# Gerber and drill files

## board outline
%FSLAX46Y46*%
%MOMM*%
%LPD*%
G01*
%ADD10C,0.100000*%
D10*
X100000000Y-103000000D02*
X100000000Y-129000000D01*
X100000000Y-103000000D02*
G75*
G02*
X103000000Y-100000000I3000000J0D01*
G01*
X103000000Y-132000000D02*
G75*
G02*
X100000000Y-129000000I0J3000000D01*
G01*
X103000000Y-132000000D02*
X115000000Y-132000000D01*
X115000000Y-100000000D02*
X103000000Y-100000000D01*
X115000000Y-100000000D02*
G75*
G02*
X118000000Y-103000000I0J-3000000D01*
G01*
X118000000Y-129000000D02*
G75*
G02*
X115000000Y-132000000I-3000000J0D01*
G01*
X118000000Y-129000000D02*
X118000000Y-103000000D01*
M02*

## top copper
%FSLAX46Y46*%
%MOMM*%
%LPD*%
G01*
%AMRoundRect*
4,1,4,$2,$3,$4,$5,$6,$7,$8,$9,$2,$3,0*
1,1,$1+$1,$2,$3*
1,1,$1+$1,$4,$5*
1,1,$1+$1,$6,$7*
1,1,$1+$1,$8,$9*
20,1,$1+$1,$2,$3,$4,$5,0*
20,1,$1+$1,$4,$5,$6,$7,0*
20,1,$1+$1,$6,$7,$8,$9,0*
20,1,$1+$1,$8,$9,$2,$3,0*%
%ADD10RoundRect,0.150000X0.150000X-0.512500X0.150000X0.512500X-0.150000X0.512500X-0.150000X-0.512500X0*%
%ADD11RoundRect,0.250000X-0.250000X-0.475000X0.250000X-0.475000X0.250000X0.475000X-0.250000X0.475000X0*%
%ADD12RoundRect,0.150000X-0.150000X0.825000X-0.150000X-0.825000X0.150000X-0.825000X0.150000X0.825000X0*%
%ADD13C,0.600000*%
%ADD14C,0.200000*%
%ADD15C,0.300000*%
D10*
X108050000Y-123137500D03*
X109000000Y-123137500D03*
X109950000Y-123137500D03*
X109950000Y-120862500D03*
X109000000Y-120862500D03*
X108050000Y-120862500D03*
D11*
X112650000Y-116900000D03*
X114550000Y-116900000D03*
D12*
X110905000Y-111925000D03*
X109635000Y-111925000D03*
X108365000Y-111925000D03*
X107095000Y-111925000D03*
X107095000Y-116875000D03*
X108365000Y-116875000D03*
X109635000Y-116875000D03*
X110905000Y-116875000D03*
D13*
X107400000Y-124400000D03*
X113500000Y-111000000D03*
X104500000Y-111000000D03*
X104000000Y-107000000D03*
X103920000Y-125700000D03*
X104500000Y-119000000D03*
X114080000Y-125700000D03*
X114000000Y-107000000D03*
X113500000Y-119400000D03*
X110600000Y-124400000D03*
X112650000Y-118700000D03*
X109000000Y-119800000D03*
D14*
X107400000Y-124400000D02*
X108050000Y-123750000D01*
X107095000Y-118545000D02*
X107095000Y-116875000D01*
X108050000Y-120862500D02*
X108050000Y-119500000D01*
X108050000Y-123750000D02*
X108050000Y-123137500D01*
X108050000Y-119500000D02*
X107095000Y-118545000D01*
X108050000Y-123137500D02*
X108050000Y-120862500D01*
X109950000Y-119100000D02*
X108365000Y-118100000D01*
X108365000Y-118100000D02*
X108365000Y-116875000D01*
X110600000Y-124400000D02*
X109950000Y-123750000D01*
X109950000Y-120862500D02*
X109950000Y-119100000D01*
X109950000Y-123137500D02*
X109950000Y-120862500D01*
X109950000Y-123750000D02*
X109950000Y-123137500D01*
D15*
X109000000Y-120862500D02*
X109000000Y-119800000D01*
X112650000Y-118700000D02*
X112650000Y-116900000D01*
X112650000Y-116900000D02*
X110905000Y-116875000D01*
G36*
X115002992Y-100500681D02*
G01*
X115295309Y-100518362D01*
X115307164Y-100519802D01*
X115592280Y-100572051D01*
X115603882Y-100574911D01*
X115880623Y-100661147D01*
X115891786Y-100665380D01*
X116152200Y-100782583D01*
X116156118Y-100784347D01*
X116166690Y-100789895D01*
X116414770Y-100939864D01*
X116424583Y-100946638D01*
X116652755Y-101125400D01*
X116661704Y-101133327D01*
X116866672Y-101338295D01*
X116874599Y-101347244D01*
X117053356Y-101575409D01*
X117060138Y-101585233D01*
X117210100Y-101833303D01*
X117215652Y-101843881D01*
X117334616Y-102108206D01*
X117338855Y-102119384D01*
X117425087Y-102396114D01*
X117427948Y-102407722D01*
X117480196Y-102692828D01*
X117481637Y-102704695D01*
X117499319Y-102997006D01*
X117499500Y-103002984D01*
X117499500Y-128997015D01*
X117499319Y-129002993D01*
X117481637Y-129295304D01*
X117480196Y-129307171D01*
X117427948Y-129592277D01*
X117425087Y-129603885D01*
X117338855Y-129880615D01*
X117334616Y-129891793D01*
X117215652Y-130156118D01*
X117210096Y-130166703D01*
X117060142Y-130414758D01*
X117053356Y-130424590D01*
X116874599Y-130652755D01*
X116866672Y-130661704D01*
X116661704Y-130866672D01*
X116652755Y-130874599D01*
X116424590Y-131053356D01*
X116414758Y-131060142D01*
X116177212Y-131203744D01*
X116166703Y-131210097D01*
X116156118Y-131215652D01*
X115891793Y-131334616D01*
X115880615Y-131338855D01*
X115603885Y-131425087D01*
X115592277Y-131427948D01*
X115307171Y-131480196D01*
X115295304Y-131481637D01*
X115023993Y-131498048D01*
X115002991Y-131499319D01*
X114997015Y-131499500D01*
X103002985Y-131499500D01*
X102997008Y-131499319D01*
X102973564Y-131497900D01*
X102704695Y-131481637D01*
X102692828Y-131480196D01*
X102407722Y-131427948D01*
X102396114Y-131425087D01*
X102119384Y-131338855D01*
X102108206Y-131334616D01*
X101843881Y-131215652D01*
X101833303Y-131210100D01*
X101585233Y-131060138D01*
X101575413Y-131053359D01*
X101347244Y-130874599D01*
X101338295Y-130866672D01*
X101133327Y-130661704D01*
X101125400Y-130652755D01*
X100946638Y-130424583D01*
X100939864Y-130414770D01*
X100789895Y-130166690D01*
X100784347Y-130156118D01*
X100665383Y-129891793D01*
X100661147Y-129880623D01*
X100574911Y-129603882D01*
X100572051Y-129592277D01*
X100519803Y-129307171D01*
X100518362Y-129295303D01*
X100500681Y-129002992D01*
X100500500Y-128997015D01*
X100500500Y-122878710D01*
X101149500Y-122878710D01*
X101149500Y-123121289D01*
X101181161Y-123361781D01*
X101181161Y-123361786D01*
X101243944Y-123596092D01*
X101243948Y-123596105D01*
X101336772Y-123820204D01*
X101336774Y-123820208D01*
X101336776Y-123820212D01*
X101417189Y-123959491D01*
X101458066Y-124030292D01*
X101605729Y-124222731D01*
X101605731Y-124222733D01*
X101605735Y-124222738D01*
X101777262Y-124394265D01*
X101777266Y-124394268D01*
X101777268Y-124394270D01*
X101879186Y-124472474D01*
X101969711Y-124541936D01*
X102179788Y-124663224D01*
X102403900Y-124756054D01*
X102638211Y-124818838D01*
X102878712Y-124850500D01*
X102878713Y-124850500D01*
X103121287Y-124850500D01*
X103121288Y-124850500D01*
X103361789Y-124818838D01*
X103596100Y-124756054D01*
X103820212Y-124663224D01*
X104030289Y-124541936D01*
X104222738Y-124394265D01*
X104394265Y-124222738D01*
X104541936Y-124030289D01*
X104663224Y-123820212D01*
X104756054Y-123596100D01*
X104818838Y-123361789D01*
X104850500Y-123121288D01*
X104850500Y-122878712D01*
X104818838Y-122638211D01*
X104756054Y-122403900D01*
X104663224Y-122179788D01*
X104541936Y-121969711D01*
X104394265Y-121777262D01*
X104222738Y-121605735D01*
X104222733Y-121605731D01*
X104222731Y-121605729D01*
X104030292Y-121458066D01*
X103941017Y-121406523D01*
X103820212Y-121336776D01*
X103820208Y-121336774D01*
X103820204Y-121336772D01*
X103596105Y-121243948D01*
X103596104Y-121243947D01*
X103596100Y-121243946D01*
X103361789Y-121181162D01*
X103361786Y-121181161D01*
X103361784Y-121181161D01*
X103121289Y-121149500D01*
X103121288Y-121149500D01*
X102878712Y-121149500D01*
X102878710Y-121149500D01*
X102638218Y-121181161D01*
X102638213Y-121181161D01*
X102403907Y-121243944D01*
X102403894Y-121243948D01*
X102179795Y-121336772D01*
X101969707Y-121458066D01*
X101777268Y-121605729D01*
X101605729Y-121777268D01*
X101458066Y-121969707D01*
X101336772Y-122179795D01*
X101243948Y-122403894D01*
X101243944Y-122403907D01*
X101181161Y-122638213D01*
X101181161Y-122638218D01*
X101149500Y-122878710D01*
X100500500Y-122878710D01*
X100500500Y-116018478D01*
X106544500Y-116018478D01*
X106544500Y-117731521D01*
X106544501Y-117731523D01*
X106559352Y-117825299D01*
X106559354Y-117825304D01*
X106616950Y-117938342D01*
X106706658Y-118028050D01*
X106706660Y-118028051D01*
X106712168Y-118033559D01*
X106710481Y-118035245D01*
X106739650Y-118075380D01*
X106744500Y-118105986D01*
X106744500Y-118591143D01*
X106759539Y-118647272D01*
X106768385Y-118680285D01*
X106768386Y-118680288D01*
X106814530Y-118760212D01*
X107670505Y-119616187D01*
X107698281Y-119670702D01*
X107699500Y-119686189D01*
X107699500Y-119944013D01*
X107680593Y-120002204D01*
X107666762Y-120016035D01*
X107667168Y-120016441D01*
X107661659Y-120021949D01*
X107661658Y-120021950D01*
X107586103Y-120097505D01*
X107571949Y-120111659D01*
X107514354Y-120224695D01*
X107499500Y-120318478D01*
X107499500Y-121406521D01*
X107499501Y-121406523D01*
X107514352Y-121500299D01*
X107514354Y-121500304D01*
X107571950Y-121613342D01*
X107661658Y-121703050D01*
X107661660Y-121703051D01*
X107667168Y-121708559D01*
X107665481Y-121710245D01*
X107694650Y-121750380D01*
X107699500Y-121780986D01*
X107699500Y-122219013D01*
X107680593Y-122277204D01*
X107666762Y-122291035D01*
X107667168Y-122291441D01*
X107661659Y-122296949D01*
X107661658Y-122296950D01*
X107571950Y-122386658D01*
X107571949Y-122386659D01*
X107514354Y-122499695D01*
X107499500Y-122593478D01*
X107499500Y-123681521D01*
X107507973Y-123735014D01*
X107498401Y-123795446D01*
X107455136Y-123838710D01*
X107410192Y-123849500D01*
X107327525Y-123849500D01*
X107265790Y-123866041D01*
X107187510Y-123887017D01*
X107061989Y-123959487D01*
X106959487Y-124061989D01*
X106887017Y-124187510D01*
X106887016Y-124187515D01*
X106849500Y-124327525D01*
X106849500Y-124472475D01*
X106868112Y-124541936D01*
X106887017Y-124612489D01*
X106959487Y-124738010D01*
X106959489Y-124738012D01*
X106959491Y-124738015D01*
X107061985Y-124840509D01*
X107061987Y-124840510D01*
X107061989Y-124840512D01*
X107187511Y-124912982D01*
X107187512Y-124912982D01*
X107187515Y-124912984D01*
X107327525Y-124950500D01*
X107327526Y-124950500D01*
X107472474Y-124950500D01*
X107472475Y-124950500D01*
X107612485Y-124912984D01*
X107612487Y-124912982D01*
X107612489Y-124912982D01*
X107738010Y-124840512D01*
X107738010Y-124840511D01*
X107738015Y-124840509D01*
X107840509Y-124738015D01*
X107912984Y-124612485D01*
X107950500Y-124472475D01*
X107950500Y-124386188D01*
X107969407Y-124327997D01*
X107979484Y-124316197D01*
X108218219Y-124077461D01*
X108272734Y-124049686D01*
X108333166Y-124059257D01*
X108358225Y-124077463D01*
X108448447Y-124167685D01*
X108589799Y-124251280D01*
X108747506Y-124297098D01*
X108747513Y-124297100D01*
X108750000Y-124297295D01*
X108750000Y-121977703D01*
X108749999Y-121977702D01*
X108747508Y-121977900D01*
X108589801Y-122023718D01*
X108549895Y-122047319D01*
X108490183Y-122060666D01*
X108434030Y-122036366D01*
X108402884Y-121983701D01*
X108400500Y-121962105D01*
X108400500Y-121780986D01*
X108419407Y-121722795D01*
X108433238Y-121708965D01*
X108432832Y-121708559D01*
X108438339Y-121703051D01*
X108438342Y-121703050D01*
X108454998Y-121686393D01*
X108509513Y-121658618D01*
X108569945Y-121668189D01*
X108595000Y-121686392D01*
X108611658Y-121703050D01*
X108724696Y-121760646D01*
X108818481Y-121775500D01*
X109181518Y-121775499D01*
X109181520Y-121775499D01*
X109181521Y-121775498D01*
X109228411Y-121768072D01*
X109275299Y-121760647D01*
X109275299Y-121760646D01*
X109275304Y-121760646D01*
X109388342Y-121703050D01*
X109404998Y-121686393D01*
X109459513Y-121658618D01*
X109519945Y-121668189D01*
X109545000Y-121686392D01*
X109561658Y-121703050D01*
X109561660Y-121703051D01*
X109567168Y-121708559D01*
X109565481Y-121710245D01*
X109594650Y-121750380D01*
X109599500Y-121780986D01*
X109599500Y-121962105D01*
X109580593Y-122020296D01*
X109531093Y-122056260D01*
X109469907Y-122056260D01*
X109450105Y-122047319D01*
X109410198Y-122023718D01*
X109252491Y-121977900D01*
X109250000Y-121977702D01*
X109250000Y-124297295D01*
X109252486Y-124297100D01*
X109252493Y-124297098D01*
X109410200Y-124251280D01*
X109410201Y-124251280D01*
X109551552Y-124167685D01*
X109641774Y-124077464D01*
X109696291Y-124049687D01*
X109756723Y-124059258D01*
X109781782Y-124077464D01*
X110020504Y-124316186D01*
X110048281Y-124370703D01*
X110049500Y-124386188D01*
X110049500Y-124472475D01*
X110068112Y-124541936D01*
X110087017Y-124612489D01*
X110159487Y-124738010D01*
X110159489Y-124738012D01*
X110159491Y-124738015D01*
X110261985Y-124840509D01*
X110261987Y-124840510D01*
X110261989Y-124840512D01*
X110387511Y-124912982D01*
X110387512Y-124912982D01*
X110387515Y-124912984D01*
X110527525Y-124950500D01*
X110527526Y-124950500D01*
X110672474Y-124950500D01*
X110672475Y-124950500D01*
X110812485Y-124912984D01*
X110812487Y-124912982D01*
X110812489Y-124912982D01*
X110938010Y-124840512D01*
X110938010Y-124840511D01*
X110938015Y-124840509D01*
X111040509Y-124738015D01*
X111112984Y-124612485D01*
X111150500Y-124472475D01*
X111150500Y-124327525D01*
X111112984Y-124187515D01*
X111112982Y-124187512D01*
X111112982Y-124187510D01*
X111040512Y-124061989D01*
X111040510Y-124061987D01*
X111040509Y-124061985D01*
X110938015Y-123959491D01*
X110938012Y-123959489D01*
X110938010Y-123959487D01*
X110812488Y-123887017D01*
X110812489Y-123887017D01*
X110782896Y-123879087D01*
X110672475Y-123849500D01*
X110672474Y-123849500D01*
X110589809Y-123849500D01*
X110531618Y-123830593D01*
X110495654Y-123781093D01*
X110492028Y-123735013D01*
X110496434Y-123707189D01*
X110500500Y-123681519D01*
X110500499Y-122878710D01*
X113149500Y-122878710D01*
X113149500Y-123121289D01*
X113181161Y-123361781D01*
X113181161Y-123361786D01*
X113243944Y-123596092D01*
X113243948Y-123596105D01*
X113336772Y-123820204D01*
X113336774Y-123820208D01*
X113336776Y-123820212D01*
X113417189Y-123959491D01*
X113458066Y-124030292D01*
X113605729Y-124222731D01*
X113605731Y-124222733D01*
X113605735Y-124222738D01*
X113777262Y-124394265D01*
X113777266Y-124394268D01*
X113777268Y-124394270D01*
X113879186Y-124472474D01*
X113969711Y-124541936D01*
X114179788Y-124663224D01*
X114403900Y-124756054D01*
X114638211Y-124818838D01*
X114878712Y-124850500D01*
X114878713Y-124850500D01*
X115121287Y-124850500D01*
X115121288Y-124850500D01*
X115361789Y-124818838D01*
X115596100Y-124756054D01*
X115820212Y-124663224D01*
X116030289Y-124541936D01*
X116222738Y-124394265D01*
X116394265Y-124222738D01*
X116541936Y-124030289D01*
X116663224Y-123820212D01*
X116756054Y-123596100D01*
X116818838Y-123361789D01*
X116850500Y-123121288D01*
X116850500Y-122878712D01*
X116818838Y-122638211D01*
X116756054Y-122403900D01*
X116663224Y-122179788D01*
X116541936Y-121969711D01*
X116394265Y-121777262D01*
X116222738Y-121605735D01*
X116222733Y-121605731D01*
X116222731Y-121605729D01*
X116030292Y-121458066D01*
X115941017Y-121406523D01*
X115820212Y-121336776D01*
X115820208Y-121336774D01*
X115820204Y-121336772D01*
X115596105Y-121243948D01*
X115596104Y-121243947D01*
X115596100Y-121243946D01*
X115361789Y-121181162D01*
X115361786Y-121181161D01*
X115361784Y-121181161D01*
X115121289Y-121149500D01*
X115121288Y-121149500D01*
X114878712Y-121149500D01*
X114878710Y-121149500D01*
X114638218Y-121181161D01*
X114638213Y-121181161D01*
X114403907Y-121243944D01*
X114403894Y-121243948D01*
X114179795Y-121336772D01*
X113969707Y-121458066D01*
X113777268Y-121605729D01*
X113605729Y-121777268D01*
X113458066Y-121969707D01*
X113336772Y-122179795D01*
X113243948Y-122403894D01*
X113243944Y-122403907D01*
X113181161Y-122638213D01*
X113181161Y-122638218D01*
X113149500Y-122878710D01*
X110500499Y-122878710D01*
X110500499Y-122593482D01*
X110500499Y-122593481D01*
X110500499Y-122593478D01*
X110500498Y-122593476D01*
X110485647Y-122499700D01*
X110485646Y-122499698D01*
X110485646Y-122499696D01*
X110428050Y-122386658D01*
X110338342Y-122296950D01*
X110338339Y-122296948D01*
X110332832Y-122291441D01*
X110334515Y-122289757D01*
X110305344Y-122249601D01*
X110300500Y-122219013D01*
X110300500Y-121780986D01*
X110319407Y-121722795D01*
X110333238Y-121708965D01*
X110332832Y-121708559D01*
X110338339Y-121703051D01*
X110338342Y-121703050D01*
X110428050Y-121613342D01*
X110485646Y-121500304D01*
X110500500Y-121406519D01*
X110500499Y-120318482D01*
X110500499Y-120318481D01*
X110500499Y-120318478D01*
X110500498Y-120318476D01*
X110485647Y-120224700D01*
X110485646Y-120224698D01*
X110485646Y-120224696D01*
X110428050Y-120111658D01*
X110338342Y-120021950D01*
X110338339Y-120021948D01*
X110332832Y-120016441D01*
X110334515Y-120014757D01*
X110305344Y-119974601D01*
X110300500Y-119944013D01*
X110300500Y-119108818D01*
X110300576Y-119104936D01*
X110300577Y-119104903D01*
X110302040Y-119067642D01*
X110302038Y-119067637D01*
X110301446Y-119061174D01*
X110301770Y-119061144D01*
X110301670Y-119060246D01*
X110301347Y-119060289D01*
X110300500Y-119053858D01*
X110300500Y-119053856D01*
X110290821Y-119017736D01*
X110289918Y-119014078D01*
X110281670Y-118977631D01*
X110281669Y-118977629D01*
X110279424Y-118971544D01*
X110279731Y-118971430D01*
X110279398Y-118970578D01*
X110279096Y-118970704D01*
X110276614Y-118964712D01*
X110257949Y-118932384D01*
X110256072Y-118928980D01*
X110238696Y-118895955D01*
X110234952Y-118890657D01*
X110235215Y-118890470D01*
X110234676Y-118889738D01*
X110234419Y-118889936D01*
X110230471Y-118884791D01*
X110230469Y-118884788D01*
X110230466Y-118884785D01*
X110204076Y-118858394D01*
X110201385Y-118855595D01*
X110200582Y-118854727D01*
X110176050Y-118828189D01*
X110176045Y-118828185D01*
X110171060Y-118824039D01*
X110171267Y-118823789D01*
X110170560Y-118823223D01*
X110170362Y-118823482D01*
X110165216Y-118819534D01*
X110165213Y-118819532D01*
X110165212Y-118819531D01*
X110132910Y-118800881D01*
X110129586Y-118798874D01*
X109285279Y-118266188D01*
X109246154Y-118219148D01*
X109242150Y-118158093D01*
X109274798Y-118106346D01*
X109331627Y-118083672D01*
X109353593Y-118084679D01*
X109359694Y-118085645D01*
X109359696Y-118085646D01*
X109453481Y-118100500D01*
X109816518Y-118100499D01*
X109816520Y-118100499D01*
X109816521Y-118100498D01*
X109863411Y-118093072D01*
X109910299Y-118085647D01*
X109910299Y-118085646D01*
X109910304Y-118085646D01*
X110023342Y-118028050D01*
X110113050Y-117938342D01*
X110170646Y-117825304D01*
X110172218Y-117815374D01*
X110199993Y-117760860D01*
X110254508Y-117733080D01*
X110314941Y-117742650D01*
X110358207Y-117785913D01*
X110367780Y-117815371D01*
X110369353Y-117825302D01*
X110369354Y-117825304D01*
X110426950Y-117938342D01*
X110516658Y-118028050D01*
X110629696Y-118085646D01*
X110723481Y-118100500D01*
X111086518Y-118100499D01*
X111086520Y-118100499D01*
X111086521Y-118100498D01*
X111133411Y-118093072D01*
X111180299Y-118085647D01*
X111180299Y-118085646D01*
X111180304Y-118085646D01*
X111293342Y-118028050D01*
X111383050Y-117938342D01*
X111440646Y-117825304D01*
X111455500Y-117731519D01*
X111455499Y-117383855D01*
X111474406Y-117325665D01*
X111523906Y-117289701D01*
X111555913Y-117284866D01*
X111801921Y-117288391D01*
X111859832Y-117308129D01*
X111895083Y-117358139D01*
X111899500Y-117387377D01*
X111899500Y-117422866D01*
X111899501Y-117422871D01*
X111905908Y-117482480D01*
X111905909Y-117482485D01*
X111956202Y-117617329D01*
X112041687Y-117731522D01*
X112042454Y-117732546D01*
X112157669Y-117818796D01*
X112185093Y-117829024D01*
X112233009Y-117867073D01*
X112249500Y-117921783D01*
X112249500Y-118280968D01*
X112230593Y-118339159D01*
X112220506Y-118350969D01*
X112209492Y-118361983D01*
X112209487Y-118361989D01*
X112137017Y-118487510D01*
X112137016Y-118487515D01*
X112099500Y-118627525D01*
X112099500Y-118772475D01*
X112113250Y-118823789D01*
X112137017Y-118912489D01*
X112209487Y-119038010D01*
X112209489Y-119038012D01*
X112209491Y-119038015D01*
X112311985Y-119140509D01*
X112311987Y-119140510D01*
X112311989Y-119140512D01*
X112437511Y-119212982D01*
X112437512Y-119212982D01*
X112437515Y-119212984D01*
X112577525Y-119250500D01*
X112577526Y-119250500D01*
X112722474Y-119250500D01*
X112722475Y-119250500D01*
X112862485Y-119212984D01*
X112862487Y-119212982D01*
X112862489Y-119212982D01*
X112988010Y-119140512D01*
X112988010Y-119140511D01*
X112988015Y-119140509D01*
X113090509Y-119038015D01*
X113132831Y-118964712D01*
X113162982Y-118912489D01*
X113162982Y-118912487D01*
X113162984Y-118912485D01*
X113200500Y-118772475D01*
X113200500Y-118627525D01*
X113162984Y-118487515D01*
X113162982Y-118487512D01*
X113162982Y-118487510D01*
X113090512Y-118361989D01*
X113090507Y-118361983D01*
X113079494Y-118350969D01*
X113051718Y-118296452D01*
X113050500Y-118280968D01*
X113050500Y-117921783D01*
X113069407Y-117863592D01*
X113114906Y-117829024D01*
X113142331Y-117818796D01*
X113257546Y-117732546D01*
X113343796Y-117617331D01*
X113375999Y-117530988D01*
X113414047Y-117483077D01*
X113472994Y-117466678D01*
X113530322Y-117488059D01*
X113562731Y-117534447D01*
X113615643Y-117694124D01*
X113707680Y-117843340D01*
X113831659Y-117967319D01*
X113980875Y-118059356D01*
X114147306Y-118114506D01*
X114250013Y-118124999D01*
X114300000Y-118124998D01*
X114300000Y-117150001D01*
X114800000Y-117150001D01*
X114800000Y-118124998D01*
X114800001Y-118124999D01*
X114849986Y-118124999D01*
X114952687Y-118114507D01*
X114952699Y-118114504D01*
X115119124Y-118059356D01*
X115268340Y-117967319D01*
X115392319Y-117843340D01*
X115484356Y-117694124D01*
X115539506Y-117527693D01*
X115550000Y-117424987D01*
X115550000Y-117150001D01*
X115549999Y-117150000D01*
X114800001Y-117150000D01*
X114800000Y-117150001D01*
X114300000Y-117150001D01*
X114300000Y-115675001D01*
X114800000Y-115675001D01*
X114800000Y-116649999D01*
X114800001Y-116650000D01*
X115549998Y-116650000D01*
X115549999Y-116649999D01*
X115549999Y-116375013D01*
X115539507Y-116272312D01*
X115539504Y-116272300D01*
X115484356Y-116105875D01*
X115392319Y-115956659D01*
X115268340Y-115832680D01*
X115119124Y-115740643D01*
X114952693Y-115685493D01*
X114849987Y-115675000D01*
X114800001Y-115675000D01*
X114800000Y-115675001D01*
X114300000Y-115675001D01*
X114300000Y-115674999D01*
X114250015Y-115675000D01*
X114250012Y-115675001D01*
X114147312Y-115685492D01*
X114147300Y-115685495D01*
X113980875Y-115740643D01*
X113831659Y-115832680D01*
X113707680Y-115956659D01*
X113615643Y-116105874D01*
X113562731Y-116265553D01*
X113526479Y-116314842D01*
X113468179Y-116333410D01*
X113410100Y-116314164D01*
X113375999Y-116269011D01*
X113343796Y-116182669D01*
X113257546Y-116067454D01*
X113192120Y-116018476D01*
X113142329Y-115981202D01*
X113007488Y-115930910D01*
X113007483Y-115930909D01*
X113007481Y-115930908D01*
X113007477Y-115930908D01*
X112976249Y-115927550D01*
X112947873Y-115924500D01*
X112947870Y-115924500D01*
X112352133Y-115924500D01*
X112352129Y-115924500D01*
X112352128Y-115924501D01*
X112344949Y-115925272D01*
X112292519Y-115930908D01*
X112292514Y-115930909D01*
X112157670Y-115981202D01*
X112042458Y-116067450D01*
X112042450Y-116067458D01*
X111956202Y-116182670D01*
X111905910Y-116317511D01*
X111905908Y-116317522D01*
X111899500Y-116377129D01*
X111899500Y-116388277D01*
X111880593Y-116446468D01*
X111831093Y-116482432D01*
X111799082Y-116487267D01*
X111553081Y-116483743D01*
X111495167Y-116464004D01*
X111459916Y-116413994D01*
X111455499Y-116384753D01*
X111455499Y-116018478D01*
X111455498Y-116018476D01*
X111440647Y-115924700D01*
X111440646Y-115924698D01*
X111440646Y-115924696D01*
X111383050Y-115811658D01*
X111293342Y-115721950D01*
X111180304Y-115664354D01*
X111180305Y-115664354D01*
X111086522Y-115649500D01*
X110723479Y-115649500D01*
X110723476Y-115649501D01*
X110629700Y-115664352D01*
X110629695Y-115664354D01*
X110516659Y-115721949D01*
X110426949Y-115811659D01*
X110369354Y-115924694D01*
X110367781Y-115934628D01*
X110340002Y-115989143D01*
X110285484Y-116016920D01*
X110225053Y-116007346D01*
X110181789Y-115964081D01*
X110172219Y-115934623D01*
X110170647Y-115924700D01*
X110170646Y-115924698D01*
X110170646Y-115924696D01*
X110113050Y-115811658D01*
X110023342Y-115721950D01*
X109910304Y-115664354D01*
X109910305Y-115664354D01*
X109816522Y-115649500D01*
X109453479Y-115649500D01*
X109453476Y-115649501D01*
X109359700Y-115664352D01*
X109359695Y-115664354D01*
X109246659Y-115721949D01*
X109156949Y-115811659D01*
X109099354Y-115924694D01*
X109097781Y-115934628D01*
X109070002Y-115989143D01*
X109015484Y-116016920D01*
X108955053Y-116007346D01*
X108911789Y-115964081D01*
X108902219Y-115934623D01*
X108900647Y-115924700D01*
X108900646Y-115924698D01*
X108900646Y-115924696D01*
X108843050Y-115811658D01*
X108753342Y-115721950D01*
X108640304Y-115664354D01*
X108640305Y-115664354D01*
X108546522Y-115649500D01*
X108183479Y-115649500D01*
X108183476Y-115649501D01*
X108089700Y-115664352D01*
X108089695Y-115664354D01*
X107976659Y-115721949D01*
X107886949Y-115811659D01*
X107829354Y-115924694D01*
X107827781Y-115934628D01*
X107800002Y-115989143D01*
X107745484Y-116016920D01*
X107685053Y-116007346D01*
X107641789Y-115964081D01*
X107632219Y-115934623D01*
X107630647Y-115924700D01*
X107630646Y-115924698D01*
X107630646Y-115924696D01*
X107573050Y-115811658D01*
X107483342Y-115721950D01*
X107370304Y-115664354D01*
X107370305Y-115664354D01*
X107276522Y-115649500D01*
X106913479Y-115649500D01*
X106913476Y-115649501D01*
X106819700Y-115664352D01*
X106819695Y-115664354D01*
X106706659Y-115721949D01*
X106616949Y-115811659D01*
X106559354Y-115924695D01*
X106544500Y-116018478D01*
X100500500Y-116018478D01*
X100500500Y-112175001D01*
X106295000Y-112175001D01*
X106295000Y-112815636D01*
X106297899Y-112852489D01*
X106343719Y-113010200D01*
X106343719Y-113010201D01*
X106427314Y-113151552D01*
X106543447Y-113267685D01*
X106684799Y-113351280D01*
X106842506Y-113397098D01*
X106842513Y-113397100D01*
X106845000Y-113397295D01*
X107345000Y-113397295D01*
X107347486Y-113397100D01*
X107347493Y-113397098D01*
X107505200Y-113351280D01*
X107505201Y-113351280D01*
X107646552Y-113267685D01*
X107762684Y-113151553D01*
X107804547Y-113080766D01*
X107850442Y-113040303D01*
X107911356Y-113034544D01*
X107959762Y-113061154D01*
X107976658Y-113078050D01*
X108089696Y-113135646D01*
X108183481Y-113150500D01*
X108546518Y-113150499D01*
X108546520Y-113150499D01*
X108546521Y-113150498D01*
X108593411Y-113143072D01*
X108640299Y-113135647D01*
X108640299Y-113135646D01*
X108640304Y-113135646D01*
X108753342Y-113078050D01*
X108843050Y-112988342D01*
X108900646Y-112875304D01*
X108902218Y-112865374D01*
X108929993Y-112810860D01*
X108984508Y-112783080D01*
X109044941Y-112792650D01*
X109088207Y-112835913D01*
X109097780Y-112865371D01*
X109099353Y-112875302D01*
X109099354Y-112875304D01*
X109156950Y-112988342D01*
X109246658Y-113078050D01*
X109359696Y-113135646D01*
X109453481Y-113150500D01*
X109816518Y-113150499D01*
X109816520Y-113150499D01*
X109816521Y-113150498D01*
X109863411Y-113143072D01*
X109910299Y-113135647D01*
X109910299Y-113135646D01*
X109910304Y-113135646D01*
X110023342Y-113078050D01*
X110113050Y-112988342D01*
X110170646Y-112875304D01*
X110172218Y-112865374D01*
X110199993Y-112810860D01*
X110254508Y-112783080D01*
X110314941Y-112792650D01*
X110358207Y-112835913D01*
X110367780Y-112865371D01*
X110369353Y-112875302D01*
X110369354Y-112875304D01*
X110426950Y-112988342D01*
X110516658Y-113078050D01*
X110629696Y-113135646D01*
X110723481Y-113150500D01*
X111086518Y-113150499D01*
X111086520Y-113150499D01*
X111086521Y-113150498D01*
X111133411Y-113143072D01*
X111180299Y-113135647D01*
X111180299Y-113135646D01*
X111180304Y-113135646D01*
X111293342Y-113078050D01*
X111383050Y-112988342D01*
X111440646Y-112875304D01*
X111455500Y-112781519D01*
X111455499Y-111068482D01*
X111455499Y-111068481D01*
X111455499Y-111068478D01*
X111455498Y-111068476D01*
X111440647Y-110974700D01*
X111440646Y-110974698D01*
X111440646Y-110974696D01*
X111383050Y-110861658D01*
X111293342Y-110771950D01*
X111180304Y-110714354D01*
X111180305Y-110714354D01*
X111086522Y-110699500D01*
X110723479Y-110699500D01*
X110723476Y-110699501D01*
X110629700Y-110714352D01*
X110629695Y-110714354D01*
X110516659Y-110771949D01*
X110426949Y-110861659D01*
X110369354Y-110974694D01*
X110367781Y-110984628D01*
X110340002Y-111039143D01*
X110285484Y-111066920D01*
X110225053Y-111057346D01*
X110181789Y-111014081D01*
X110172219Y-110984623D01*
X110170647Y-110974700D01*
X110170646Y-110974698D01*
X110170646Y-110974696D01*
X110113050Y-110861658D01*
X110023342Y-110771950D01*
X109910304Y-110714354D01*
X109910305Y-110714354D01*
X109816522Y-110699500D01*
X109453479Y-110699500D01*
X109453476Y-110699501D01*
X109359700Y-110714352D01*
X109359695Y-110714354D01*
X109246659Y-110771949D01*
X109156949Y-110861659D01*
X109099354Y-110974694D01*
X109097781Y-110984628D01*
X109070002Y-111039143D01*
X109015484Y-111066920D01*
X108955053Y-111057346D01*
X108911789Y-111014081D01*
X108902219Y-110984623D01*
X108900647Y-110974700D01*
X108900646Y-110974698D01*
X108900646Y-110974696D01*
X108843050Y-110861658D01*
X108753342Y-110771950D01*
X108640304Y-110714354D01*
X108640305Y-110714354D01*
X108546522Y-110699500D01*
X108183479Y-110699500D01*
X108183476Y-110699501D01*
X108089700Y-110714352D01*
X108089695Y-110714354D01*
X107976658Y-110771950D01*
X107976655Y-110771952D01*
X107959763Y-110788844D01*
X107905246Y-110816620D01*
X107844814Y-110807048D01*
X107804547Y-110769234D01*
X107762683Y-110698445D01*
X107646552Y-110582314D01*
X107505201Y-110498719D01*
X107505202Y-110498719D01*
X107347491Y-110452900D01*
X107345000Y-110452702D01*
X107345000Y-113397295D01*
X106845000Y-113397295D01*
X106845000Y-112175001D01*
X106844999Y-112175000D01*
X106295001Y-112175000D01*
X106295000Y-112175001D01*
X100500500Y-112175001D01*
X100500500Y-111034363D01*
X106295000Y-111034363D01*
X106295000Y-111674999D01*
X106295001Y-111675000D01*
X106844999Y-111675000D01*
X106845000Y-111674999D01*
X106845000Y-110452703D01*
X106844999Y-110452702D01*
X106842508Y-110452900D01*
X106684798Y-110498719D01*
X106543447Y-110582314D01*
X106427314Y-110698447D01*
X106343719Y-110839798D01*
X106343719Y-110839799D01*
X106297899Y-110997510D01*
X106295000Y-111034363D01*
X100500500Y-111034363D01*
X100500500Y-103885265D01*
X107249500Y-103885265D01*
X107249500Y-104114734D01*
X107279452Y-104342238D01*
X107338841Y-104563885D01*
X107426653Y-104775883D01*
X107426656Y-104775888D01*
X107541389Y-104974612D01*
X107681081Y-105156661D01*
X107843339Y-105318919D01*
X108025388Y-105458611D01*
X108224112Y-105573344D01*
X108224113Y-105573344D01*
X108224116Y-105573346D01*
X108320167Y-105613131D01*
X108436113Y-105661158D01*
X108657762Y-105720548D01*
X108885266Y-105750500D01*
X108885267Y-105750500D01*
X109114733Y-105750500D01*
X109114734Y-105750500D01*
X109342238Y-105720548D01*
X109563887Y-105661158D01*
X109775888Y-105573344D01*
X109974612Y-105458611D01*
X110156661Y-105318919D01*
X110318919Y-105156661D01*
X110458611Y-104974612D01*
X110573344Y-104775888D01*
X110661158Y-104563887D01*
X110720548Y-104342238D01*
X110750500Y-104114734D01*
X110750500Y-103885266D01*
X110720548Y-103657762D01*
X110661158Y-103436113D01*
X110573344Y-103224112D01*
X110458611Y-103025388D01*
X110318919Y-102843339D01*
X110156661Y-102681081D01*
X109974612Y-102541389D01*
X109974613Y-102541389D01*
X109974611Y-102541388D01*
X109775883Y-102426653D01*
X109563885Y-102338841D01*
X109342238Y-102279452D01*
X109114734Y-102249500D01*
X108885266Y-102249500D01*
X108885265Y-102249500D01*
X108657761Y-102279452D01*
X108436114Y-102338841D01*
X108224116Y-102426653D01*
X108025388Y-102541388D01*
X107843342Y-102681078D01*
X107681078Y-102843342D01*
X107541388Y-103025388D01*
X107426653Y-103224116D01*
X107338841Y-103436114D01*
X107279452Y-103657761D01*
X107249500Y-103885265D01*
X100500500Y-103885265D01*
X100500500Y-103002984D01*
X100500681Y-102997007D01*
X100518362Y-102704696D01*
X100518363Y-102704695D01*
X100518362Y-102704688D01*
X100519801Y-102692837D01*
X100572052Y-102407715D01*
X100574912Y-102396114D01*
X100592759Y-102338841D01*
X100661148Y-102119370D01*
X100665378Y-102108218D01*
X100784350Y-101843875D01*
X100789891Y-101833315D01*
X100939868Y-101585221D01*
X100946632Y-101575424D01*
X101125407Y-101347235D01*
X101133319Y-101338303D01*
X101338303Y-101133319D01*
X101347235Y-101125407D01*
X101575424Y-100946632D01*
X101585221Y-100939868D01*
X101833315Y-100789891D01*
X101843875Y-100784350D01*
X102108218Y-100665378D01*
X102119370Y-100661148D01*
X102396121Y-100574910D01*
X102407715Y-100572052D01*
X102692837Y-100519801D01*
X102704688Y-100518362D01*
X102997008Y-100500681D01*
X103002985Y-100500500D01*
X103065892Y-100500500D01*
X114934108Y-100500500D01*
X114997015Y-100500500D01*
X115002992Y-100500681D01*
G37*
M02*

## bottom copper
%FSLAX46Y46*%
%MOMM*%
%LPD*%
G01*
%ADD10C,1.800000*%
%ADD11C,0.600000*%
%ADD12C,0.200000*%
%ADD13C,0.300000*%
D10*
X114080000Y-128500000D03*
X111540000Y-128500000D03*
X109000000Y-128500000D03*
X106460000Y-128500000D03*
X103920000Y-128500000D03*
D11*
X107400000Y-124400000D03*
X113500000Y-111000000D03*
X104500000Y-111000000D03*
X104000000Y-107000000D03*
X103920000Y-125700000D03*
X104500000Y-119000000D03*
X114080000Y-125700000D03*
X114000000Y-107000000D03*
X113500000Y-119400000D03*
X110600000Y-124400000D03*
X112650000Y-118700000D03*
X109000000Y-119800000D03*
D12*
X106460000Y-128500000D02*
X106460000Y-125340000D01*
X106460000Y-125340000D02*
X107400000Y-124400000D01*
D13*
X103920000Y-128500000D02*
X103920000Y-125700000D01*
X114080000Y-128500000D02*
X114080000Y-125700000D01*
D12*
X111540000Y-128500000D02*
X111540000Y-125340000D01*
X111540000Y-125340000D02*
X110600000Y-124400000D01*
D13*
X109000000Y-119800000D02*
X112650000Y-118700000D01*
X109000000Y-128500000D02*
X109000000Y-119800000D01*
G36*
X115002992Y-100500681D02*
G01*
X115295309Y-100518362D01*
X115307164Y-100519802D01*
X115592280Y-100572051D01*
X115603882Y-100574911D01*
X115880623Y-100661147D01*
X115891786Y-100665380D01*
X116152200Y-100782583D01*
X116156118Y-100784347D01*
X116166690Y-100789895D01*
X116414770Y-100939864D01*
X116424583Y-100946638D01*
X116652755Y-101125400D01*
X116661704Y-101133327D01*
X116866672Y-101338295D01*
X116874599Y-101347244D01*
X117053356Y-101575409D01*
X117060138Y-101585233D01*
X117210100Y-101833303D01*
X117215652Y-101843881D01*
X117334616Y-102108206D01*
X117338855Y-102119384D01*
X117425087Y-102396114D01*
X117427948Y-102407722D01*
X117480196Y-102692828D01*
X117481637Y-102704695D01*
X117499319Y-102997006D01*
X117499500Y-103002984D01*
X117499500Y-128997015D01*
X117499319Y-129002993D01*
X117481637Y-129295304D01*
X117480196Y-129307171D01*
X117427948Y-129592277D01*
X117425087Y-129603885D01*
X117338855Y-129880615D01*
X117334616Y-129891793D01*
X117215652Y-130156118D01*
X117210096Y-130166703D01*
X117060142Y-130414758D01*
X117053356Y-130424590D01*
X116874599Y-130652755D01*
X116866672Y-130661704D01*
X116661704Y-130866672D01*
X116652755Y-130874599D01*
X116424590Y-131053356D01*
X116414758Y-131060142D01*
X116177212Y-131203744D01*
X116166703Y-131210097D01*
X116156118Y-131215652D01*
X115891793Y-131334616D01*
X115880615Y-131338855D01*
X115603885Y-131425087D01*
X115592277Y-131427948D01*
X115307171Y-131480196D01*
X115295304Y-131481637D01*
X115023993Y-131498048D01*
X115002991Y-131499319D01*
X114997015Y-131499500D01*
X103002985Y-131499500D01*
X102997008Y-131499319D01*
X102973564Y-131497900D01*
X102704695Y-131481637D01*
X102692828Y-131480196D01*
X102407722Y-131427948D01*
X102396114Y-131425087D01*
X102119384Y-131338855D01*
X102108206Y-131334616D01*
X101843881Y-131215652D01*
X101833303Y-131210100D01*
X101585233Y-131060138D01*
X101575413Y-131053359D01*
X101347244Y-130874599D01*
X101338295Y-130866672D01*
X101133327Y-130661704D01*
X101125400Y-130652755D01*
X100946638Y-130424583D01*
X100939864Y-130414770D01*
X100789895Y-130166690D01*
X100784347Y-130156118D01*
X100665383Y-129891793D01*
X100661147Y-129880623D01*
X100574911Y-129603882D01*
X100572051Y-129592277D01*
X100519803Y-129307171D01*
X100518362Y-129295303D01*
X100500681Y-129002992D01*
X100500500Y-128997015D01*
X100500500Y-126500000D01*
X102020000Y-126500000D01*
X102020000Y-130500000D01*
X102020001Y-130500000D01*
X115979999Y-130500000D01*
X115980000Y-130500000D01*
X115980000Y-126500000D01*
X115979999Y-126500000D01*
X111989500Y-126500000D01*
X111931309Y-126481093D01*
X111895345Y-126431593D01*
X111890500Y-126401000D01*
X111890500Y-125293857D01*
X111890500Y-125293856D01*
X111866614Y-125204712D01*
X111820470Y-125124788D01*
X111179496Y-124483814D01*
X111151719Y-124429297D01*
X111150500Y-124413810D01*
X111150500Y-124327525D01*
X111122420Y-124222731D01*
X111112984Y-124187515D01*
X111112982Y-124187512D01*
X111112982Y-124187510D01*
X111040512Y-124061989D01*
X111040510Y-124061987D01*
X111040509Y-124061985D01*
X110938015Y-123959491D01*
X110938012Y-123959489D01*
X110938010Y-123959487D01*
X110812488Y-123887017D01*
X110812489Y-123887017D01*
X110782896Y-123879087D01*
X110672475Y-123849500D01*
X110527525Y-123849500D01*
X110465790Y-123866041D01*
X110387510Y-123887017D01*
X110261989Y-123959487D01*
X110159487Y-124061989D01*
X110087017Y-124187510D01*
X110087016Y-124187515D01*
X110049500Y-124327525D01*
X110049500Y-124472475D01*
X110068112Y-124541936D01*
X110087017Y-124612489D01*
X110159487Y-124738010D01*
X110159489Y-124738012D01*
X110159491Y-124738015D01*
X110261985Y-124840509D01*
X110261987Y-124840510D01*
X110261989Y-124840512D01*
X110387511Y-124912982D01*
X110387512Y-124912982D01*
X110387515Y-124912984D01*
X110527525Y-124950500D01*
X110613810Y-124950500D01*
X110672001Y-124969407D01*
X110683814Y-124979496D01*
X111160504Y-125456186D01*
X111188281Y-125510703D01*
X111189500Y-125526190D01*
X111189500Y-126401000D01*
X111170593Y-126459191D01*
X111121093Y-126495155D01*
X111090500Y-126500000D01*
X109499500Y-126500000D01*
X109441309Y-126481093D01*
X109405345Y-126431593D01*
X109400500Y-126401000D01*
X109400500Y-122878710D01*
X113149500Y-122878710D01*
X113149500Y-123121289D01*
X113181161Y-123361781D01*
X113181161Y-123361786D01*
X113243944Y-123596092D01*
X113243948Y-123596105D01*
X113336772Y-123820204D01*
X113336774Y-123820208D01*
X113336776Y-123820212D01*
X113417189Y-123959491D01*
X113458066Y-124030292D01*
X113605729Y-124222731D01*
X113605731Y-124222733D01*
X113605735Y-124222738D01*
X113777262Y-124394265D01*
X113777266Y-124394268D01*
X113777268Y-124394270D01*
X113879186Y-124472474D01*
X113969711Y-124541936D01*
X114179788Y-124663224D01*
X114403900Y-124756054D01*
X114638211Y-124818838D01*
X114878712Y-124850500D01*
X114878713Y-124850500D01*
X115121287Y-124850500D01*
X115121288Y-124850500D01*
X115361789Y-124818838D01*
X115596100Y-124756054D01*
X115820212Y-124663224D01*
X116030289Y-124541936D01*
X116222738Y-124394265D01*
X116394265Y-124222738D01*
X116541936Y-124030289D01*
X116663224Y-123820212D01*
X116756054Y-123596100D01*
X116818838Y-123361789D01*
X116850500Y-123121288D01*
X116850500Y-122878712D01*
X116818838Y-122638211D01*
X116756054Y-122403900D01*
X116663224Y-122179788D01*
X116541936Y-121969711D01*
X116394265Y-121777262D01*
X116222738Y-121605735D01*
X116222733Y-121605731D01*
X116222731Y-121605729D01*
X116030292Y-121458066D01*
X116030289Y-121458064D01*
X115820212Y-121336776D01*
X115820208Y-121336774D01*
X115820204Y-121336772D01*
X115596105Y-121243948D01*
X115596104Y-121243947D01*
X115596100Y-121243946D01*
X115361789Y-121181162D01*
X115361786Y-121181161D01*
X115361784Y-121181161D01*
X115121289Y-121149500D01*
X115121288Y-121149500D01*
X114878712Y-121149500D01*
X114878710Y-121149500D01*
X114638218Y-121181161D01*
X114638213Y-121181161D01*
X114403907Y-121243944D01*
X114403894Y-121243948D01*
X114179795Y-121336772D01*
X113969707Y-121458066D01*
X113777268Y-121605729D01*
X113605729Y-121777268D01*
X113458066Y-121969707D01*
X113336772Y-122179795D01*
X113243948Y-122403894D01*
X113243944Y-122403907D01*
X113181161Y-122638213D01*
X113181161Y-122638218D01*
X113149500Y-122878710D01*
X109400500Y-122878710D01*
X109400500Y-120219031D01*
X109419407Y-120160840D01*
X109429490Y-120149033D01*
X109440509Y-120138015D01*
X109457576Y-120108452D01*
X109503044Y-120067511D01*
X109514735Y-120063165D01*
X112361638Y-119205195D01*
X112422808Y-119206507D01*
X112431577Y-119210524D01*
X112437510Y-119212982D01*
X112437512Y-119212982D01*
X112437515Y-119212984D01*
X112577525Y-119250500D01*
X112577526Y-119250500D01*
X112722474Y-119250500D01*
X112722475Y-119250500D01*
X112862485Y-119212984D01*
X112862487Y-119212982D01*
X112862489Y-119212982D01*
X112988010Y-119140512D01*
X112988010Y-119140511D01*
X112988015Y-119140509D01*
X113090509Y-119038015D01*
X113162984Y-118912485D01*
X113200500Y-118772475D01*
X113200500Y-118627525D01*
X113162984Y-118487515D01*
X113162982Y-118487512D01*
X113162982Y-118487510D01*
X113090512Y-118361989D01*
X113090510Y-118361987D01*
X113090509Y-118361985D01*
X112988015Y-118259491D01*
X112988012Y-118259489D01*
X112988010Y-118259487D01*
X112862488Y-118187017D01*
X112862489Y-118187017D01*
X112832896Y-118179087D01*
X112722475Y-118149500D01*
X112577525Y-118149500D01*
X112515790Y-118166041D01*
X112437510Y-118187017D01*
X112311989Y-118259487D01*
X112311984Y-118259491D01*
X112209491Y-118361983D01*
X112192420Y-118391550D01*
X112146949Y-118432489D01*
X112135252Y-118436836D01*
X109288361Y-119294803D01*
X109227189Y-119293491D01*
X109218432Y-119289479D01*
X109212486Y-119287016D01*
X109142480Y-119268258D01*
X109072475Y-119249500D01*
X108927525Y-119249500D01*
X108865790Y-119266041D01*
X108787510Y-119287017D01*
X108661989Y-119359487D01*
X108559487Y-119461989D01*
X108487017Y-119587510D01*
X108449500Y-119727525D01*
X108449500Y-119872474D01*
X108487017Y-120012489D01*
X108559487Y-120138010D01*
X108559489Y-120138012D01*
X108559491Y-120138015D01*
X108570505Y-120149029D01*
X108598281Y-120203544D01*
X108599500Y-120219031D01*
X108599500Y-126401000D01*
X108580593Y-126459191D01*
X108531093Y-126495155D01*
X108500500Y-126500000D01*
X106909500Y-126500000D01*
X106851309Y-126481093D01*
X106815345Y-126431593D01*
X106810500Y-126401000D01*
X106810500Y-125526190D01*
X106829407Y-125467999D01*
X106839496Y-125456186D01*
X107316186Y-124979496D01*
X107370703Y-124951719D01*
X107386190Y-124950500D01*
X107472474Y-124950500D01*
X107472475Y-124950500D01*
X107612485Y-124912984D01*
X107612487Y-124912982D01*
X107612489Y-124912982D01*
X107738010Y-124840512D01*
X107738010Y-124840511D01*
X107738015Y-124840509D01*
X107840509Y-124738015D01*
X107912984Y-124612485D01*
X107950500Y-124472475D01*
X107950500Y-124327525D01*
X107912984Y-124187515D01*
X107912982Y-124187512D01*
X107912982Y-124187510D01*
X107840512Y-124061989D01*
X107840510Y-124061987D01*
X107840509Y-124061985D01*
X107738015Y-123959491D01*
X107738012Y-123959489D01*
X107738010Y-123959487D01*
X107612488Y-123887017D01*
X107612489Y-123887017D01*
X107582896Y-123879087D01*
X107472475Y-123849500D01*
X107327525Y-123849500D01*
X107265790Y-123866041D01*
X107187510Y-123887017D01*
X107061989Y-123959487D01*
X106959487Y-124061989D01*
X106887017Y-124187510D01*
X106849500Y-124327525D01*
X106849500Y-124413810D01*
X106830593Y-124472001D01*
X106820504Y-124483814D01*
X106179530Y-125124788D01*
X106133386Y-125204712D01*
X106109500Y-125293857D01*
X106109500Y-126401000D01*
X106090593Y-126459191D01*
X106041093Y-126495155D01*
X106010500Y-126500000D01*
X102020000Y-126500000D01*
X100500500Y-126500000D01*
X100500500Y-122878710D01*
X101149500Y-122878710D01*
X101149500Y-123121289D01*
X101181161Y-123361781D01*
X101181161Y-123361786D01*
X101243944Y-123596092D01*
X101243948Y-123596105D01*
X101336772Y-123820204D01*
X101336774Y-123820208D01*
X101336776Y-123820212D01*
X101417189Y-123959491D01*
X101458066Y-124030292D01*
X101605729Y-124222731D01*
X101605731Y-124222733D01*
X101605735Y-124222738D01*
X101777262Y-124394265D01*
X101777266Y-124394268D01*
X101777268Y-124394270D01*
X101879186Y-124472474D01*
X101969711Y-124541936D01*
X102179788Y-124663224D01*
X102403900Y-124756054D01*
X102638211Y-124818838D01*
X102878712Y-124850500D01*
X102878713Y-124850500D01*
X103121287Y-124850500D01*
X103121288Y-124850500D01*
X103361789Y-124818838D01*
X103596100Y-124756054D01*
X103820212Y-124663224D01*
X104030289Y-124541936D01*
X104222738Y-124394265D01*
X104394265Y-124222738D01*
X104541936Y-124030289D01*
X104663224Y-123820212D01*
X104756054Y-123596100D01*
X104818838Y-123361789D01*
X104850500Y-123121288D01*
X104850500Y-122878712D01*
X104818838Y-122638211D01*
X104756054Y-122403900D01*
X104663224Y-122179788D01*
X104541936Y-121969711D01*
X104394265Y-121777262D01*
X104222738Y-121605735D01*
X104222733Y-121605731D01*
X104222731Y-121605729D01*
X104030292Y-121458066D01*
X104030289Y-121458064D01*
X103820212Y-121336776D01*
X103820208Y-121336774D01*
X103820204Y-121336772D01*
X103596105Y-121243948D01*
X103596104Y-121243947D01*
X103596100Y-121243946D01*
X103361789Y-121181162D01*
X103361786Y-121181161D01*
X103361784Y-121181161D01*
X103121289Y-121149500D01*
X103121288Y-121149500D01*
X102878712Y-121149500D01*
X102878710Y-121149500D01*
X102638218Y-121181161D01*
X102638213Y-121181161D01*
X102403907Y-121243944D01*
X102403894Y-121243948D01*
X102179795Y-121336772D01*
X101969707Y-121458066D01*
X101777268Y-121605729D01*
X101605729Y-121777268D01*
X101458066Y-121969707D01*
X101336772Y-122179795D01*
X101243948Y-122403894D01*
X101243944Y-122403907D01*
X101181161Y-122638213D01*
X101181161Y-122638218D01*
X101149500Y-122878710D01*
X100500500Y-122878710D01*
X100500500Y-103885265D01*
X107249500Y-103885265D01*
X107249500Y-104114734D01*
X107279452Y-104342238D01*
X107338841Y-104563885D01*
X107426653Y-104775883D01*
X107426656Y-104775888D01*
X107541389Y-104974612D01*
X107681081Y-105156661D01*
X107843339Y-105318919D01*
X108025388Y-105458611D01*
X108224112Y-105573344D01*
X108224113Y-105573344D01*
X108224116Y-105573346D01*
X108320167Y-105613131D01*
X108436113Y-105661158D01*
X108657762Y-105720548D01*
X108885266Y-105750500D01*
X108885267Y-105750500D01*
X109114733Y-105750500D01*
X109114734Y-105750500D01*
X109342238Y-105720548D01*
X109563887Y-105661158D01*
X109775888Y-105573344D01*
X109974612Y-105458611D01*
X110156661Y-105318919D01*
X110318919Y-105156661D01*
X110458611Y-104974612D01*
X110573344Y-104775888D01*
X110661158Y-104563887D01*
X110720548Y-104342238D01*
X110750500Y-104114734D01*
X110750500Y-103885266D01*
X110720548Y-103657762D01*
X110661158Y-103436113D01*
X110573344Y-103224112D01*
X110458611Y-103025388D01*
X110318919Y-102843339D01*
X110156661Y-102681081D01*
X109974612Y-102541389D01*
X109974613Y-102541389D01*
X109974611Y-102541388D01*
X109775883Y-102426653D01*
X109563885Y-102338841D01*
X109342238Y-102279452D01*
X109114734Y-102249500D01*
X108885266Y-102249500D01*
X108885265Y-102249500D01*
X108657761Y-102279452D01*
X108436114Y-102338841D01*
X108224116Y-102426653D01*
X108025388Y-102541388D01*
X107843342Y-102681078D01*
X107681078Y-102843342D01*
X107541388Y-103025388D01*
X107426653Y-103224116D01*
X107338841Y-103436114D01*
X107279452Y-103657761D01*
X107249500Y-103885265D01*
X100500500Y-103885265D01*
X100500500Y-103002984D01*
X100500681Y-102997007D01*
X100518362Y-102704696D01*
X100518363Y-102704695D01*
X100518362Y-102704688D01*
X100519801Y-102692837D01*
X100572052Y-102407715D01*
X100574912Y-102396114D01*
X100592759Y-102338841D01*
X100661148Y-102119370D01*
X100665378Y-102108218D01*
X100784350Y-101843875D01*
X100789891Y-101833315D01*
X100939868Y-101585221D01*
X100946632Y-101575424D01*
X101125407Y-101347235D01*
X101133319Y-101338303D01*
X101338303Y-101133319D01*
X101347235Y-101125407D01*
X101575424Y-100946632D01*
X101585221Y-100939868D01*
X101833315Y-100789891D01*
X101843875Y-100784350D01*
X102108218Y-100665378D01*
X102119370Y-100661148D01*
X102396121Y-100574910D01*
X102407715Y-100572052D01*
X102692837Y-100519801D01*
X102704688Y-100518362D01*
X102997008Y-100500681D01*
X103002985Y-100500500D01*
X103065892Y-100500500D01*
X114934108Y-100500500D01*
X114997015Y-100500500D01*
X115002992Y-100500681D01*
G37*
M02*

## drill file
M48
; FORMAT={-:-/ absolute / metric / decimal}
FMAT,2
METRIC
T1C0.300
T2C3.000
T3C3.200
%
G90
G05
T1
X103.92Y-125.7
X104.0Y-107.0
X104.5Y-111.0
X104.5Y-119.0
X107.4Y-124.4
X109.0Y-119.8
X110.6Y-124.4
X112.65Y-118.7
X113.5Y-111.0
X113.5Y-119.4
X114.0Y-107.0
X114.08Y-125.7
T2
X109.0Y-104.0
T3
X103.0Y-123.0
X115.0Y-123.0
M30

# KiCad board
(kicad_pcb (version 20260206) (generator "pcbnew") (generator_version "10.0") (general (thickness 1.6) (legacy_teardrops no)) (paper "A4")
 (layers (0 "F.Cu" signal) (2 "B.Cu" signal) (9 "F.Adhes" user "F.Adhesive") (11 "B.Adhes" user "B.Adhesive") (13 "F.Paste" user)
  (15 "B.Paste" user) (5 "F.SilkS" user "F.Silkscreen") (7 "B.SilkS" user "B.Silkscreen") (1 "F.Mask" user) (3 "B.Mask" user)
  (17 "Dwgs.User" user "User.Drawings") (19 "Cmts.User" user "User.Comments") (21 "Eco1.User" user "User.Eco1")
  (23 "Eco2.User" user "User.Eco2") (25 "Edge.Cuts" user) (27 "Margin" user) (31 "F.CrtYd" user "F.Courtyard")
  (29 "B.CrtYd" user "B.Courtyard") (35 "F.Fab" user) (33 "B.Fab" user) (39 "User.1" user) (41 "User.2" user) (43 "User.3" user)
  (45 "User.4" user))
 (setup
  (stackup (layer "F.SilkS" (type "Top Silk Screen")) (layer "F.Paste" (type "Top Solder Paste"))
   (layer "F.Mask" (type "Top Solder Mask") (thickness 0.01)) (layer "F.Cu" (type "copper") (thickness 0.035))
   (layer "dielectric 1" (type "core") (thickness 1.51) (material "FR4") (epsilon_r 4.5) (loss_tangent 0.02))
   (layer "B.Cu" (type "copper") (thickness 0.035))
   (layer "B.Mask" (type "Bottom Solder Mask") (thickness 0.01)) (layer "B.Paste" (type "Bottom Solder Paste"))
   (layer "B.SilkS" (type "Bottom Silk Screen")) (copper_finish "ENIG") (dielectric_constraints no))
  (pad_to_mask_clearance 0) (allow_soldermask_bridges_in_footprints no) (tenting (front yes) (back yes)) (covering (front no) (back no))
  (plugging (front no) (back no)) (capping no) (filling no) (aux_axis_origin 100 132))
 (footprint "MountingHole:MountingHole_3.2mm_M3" (layer "F.Cu") (at 103 123)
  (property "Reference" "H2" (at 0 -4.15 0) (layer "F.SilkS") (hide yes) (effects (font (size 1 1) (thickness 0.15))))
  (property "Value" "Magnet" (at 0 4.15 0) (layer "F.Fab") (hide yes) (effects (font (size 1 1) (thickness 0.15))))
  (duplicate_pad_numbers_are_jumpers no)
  (pad "" np_thru_hole circle (at 0 0) (size 3.2 3.2) (drill 3.2) (layers "*.Cu" "*.Mask")))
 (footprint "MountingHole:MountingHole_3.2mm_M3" (layer "F.Cu") (at 115 123)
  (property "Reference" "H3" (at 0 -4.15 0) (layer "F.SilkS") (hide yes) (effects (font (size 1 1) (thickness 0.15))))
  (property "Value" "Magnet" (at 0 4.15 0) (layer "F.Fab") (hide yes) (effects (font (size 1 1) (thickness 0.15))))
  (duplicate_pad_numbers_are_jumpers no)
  (pad "" np_thru_hole circle (at 0 0) (size 3.2 3.2) (drill 3.2) (layers "*.Cu" "*.Mask")))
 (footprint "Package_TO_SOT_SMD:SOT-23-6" (layer "F.Cu") (at 109 122 90)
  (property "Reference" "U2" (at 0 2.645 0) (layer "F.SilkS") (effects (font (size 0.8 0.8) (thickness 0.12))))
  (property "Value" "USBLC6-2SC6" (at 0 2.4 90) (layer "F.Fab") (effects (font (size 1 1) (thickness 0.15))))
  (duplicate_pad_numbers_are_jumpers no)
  (pad "1" smd roundrect (at -1.1375 -0.95 90) (size 1.325 0.6) (layers "F.Cu" "F.Mask" "F.Paste") (roundrect_rratio 0.25) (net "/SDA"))
  (pad "2" smd roundrect (at -1.1375 0 90) (size 1.325 0.6) (layers "F.Cu" "F.Mask" "F.Paste") (roundrect_rratio 0.25) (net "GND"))
  (pad "3" smd roundrect (at -1.1375 0.95 90) (size 1.325 0.6) (layers "F.Cu" "F.Mask" "F.Paste") (roundrect_rratio 0.25) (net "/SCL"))
  (pad "4" smd roundrect (at 1.1375 0.95 90) (size 1.325 0.6) (layers "F.Cu" "F.Mask" "F.Paste") (roundrect_rratio 0.25) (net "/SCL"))
  (pad "5" smd roundrect (at 1.1375 0 90) (size 1.325 0.6) (layers "F.Cu" "F.Mask" "F.Paste") (roundrect_rratio 0.25) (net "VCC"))
  (pad "6" smd roundrect (at 1.1375 -0.95 90) (size 1.325 0.6) (layers "F.Cu" "F.Mask" "F.Paste") (roundrect_rratio 0.25) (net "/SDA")))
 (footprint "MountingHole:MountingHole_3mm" (layer "F.Cu") (at 109 104)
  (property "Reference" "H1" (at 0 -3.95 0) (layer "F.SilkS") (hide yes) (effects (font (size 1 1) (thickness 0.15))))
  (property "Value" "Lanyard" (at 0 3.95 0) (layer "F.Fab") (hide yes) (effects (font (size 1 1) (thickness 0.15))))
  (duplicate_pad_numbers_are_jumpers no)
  (pad "" np_thru_hole circle (at 0 0) (size 3 3) (drill 3) (layers "*.Cu" "*.Mask")))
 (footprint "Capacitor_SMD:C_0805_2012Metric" (layer "F.Cu") (at 113.6 116.9)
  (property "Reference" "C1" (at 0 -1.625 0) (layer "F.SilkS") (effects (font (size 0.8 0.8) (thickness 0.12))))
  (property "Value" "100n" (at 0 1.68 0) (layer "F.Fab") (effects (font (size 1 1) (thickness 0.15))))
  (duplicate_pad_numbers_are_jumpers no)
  (pad "1" smd roundrect (at -0.95 0) (size 1 1.45) (layers "F.Cu" "F.Mask" "F.Paste") (roundrect_rratio 0.25) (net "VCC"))
  (pad "2" smd roundrect (at 0.95 0) (size 1 1.45) (layers "F.Cu" "F.Mask" "F.Paste") (roundrect_rratio 0.25) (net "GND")))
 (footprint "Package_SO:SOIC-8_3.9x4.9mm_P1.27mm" (layer "F.Cu") (at 109 114.4 -90)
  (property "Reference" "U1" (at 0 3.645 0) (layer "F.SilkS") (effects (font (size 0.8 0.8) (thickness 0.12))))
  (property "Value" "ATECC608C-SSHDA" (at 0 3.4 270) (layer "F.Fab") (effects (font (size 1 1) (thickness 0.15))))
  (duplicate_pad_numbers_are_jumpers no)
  (pad "1" smd roundrect (at -2.475 -1.905 270) (size 1.95 0.6) (layers "F.Cu" "F.Mask" "F.Paste") (roundrect_rratio 0.25)
   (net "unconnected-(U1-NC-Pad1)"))
  (pad "2" smd roundrect (at -2.475 -0.635 270) (size 1.95 0.6) (layers "F.Cu" "F.Mask" "F.Paste") (roundrect_rratio 0.25)
   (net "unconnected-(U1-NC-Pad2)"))
  (pad "3" smd roundrect (at -2.475 0.635 270) (size 1.95 0.6) (layers "F.Cu" "F.Mask" "F.Paste") (roundrect_rratio 0.25)
   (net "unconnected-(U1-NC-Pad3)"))
  (pad "4" smd roundrect (at -2.475 1.905 270) (size 1.95 0.6) (layers "F.Cu" "F.Mask" "F.Paste") (roundrect_rratio 0.25) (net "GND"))
  (pad "5" smd roundrect (at 2.475 1.905 270) (size 1.95 0.6) (layers "F.Cu" "F.Mask" "F.Paste") (roundrect_rratio 0.25) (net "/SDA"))
  (pad "6" smd roundrect (at 2.475 0.635 270) (size 1.95 0.6) (layers "F.Cu" "F.Mask" "F.Paste") (roundrect_rratio 0.25) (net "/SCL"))
  (pad "7" smd roundrect (at 2.475 -0.635 270) (size 1.95 0.6) (layers "F.Cu" "F.Mask" "F.Paste") (roundrect_rratio 0.25)
   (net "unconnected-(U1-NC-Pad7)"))
  (pad "8" smd roundrect (at 2.475 -1.905 270) (size 1.95 0.6) (layers "F.Cu" "F.Mask" "F.Paste") (roundrect_rratio 0.25) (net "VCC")))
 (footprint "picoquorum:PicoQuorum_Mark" (layer "B.Cu") (at 109 108.6 180)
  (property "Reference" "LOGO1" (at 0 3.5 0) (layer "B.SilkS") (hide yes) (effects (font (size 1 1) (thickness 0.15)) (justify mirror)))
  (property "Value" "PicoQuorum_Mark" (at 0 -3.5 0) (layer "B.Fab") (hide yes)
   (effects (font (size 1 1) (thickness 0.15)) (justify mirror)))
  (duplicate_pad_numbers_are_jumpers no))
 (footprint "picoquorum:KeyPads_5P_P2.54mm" (layer "B.Cu") (at 109 128.5 180)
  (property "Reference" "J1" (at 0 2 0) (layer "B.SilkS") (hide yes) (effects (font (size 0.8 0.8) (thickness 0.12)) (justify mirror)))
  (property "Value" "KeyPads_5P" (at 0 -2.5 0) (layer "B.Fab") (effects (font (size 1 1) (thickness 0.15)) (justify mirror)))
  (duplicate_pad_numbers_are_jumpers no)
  (pad "1" smd circle (at -5.08 0 180) (size 1.8 1.8) (layers "B.Cu" "B.Mask") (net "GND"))
  (pad "2" smd circle (at -2.54 0 180) (size 1.8 1.8) (layers "B.Cu" "B.Mask") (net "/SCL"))
  (pad "3" smd circle (at 0 0 180) (size 1.8 1.8) (layers "B.Cu" "B.Mask") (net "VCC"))
  (pad "4" smd circle (at 2.54 0 180) (size 1.8 1.8) (layers "B.Cu" "B.Mask") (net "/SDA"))
  (pad "5" smd circle (at 5.08 0 180) (size 1.8 1.8) (layers "B.Cu" "B.Mask") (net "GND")))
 (gr_line (start 100 103) (end 100 129) (stroke (width 0.1) (type default)) (layer "Edge.Cuts"))
 (gr_arc (start 100 103) (mid 100.87868 100.87868) (end 103 100) (stroke (width 0.1) (type default)) (layer "Edge.Cuts"))
 (gr_arc (start 103 132) (mid 100.87868 131.12132) (end 100 129) (stroke (width 0.1) (type default)) (layer "Edge.Cuts"))
 (gr_line (start 103 132) (end 115 132) (stroke (width 0.1) (type default)) (layer "Edge.Cuts"))
 (gr_line (start 115 100) (end 103 100) (stroke (width 0.1) (type default)) (layer "Edge.Cuts"))
 (gr_arc (start 115 100) (mid 117.12132 100.87868) (end 118 103) (stroke (width 0.1) (type default)) (layer "Edge.Cuts"))
 (gr_arc (start 118 129) (mid 117.12132 131.12132) (end 115 132) (stroke (width 0.1) (type default)) (layer "Edge.Cuts"))
 (gr_line (start 118 129) (end 118 103) (stroke (width 0.1) (type default)) (layer "Edge.Cuts"))
 (segment (start 107.4 124.4) (end 108.05 123.75) (width 0.2) (layer "F.Cu") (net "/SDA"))
 (segment (start 107.095 118.545) (end 107.095 116.875) (width 0.2) (layer "F.Cu") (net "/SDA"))
 (segment (start 108.05 120.8625) (end 108.05 119.5) (width 0.2) (layer "F.Cu") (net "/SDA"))
 (segment (start 108.05 123.75) (end 108.05 123.1375) (width 0.2) (layer "F.Cu") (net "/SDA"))
 (segment (start 108.05 119.5) (end 107.095 118.545) (width 0.2) (layer "F.Cu") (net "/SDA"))
 (segment (start 108.05 123.1375) (end 108.05 120.8625) (width 0.2) (layer "F.Cu") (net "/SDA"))
 (via (at 107.4 124.4) (size 0.6) (drill 0.3) (layers "F.Cu" "B.Cu") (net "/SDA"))
 (segment (start 106.46 128.5) (end 106.46 125.34) (width 0.2) (layer "B.Cu") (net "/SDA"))
 (segment (start 106.46 125.34) (end 107.4 124.4) (width 0.2) (layer "B.Cu") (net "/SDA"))
 (via (at 113.5 111) (size 0.6) (drill 0.3) (layers "F.Cu" "B.Cu") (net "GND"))
 (via (at 104.5 111) (size 0.6) (drill 0.3) (layers "F.Cu" "B.Cu") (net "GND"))
 (via (at 104 107) (size 0.6) (drill 0.3) (layers "F.Cu" "B.Cu") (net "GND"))
 (via (at 103.92 125.7) (size 0.6) (drill 0.3) (layers "F.Cu" "B.Cu") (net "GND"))
 (via (at 104.5 119) (size 0.6) (drill 0.3) (layers "F.Cu" "B.Cu") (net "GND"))
 (via (at 114.08 125.7) (size 0.6) (drill 0.3) (layers "F.Cu" "B.Cu") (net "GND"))
 (via (at 114 107) (size 0.6) (drill 0.3) (layers "F.Cu" "B.Cu") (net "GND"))
 (via (at 113.5 119.4) (size 0.6) (drill 0.3) (layers "F.Cu" "B.Cu") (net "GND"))
 (segment (start 103.92 128.5) (end 103.92 125.7) (width 0.3) (layer "B.Cu") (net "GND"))
 (segment (start 114.08 128.5) (end 114.08 125.7) (width 0.3) (layer "B.Cu") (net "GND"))
 (segment (start 109.95 119.1) (end 108.365 118.1) (width 0.2) (layer "F.Cu") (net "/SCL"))
 (segment (start 108.365 118.1) (end 108.365 116.875) (width 0.2) (layer "F.Cu") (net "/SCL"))
 (segment (start 110.6 124.4) (end 109.95 123.75) (width 0.2) (layer "F.Cu") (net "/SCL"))
 (segment (start 109.95 120.8625) (end 109.95 119.1) (width 0.2) (layer "F.Cu") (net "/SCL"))
 (segment (start 109.95 123.1375) (end 109.95 120.8625) (width 0.2) (layer "F.Cu") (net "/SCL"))
 (segment (start 109.95 123.75) (end 109.95 123.1375) (width 0.2) (layer "F.Cu") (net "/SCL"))
 (via (at 110.6 124.4) (size 0.6) (drill 0.3) (layers "F.Cu" "B.Cu") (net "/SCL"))
 (segment (start 111.54 128.5) (end 111.54 125.34) (width 0.2) (layer "B.Cu") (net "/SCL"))
 (segment (start 111.54 125.34) (end 110.6 124.4) (width 0.2) (layer "B.Cu") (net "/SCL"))
 (segment (start 109 120.8625) (end 109 119.8) (width 0.3) (layer "F.Cu") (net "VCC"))
 (segment (start 112.65 118.7) (end 112.65 116.9) (width 0.3) (layer "F.Cu") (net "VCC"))
 (segment (start 112.65 116.9) (end 110.905 116.875) (width 0.3) (layer "F.Cu") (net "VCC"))
 (via (at 112.65 118.7) (size 0.6) (drill 0.3) (layers "F.Cu" "B.Cu") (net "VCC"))
 (via (at 109 119.8) (size 0.6) (drill 0.3) (layers "F.Cu" "B.Cu") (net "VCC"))
 (segment (start 109 119.8) (end 112.65 118.7) (width 0.3) (layer "B.Cu") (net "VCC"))
 (segment (start 109 128.5) (end 109 119.8) (width 0.3) (layer "B.Cu") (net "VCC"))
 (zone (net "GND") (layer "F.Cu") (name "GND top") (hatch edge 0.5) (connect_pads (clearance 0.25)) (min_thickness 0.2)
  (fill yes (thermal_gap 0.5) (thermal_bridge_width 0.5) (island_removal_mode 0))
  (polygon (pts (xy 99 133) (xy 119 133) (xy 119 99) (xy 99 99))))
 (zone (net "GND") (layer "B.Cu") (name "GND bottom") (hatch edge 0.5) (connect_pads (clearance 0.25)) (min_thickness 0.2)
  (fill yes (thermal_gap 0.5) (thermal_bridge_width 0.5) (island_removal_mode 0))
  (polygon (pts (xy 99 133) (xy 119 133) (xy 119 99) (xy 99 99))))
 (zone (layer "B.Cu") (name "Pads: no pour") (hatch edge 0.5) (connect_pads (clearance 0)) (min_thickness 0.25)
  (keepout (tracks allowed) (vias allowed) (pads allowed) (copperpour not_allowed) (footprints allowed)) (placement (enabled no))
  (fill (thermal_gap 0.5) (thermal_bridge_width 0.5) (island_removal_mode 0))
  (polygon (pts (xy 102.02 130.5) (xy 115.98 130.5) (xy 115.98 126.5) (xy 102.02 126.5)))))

